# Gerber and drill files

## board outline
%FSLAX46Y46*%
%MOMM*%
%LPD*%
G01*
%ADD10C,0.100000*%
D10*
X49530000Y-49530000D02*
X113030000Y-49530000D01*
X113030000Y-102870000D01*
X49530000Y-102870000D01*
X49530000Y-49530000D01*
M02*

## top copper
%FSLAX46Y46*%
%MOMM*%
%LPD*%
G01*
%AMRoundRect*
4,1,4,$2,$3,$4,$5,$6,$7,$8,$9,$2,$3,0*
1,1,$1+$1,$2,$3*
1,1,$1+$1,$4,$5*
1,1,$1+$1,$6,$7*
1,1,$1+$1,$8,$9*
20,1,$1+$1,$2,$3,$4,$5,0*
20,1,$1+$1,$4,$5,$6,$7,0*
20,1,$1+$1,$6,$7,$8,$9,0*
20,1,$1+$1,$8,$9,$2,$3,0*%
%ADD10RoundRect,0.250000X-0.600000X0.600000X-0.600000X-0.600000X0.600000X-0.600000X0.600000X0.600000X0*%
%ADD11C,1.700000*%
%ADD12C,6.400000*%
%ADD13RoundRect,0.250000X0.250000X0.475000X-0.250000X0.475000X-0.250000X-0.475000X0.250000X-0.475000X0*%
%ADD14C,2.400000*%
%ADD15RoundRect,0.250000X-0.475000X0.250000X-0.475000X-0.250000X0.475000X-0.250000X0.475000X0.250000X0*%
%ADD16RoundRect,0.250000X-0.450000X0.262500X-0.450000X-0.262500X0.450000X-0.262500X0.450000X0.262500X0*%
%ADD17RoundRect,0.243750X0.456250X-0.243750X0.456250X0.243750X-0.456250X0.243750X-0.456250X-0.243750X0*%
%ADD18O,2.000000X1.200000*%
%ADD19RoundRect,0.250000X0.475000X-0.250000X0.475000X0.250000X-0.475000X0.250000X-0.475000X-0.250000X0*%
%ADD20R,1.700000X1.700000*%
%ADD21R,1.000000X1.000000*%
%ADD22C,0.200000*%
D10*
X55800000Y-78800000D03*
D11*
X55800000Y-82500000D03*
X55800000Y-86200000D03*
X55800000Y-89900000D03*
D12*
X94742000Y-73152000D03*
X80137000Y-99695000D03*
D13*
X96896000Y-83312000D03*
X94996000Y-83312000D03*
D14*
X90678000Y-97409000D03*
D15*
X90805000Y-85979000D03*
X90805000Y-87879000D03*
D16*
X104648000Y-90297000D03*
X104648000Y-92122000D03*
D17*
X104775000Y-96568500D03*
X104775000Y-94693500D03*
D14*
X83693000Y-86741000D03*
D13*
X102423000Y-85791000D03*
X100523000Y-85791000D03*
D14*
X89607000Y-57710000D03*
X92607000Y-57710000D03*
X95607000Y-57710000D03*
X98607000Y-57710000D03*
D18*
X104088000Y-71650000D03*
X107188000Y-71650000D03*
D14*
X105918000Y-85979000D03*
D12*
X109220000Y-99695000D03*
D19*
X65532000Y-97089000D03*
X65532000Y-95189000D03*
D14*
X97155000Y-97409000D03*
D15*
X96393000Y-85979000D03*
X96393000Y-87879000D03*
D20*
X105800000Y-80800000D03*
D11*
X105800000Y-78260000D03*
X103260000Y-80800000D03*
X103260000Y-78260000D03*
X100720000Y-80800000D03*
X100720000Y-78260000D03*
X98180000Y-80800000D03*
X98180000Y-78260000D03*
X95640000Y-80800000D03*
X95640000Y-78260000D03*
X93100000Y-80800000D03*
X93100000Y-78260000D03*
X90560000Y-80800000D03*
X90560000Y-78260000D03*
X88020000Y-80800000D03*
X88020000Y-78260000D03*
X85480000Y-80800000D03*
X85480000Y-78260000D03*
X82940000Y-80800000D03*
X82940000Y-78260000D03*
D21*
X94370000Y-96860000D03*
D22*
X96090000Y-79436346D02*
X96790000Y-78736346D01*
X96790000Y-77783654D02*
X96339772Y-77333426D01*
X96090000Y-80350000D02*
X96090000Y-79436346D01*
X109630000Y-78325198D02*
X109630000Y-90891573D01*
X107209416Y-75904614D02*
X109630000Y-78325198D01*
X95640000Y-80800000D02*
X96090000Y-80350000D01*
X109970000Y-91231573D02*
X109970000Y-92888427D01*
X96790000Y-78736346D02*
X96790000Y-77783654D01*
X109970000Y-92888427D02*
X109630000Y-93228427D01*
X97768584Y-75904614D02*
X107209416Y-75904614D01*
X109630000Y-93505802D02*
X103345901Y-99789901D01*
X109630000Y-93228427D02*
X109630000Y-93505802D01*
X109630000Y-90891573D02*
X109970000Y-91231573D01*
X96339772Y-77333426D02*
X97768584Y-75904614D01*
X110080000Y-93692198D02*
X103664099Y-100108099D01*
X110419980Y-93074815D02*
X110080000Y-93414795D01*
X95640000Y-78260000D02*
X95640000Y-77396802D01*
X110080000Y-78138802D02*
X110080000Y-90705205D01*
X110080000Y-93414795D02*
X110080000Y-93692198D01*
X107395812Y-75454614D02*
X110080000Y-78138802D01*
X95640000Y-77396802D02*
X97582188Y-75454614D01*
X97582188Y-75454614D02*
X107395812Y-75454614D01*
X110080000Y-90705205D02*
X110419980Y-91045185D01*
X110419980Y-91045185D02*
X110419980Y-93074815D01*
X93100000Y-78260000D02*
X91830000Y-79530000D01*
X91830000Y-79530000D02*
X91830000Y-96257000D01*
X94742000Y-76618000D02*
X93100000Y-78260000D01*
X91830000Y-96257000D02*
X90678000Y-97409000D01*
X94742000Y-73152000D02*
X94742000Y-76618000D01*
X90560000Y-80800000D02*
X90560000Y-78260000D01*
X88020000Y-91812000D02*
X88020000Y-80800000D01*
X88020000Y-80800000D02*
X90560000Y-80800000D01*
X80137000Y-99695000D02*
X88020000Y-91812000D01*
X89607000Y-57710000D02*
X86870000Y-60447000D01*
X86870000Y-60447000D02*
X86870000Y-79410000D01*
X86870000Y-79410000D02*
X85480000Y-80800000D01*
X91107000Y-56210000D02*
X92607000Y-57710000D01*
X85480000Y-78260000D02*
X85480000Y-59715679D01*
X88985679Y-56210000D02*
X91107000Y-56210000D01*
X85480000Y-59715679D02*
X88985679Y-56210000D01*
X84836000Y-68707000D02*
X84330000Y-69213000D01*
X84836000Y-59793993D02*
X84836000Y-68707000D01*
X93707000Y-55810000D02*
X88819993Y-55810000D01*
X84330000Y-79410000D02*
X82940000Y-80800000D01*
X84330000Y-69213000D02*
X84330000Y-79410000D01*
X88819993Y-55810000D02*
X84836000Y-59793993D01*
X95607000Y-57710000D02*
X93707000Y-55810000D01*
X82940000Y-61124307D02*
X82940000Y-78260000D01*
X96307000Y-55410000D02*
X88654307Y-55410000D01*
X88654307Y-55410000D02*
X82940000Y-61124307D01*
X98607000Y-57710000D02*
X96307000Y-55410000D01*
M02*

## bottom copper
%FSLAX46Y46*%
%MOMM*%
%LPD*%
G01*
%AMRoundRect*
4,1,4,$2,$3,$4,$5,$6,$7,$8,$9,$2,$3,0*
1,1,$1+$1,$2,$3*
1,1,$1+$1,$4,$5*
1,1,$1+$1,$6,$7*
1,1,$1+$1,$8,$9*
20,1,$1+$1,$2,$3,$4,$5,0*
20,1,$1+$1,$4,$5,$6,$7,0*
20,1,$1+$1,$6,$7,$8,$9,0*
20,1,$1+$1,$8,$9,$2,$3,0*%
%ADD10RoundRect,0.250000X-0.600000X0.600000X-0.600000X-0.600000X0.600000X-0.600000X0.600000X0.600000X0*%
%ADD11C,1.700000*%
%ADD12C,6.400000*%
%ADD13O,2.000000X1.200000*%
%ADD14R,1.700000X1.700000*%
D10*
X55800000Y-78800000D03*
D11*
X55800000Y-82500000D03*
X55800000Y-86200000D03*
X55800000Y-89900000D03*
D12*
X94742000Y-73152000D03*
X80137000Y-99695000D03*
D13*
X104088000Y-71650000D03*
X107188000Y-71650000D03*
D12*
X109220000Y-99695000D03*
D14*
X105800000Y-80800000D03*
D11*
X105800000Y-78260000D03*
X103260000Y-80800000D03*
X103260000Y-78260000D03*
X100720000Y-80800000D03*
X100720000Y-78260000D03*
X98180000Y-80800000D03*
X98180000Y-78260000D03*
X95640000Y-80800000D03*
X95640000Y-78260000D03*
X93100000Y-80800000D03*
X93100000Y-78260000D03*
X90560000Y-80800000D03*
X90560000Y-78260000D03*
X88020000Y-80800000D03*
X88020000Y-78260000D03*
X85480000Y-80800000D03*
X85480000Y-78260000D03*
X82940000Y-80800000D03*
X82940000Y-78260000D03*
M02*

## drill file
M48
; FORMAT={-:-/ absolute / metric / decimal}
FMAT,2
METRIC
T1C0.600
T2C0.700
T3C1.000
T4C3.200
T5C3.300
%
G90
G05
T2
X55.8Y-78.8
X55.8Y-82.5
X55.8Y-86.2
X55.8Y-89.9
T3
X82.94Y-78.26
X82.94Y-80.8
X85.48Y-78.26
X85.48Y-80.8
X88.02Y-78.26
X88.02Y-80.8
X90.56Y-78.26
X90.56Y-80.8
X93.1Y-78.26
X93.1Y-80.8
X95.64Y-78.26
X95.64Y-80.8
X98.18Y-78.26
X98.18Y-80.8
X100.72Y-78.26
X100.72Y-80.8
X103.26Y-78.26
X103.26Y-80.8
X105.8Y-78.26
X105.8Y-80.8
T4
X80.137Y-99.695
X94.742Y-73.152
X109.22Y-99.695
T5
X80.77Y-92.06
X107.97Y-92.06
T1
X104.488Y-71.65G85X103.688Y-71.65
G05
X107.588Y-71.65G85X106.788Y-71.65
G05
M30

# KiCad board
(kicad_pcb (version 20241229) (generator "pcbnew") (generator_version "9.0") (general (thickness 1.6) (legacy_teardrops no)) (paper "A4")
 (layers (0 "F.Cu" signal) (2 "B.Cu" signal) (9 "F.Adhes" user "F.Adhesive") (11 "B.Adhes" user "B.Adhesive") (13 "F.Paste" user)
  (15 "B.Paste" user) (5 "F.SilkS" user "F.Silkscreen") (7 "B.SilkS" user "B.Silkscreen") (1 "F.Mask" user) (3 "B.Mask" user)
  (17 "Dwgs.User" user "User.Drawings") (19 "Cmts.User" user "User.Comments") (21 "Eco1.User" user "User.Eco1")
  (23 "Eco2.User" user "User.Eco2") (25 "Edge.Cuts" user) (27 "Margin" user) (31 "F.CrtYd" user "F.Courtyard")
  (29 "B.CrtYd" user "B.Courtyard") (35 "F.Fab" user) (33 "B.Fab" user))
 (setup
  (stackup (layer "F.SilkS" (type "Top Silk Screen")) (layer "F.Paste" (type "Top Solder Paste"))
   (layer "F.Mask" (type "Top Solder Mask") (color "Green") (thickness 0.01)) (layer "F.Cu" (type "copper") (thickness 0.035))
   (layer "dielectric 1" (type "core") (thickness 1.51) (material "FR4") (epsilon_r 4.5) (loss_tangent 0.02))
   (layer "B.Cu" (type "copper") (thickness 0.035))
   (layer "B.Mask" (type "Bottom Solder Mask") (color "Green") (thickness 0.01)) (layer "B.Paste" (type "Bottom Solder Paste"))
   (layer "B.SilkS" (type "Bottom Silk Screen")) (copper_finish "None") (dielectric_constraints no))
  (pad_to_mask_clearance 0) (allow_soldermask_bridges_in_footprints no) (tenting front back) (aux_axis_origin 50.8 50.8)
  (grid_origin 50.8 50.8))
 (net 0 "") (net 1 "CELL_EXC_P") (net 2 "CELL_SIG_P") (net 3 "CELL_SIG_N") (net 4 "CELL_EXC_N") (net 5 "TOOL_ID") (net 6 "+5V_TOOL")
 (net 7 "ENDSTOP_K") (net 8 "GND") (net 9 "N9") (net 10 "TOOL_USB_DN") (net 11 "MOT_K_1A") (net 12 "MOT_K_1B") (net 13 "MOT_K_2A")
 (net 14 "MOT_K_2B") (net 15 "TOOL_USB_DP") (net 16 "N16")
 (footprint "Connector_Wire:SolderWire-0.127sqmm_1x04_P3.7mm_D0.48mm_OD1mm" (layer "F.Cu") (at 55.8 78.8 -90)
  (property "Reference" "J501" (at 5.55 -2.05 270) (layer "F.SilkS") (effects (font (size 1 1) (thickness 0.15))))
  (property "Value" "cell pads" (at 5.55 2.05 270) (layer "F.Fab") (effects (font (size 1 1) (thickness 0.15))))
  (pad "1" thru_hole roundrect (at 0 0 270) (size 1.7 1.7) (drill 0.7) (layers "*.Cu" "*.Mask") (remove_unused_layers no)
   (roundrect_rratio 0.147059) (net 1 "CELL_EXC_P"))
  (pad "2" thru_hole circle (at 3.7 0 270) (size 1.7 1.7) (drill 0.7) (layers "*.Cu" "*.Mask") (remove_unused_layers no)
   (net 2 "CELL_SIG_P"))
  (pad "3" thru_hole circle (at 7.4 0 270) (size 1.7 1.7) (drill 0.7) (layers "*.Cu" "*.Mask") (remove_unused_layers no)
   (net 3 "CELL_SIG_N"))
  (pad "4" thru_hole circle (at 11.1 0 270) (size 1.7 1.7) (drill 0.7) (layers "*.Cu" "*.Mask") (remove_unused_layers no)
   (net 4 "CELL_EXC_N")))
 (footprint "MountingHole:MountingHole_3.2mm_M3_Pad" (layer "F.Cu") (at 94.742 73.152)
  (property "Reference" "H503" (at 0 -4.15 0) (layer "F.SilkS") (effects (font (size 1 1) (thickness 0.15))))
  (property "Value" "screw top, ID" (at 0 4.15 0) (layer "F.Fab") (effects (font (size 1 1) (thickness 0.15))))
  (pad "1" thru_hole circle (at 0 0) (size 6.4 6.4) (drill 3.2) (layers "*.Cu" "*.Mask") (remove_unused_layers no) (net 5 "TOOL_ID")
   (zone_connect 2)))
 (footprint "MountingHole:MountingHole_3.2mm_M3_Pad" (layer "F.Cu") (at 80.137 99.695)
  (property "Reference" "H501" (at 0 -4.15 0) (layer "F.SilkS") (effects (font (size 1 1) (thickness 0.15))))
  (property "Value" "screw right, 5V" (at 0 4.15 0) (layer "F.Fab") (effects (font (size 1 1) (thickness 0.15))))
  (pad "1" thru_hole circle (at 0 0) (size 6.4 6.4) (drill 3.2) (layers "*.Cu" "*.Mask") (remove_unused_layers no) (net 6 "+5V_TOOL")
   (zone_connect 2)))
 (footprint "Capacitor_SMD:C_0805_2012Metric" (layer "F.Cu") (at 95.946 83.312 180)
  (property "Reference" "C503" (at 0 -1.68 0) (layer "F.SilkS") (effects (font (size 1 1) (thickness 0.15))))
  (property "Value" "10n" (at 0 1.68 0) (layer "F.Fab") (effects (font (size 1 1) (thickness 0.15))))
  (pad "1" smd roundrect (at -0.95 0 180) (size 1 1.45) (layers "F.Cu" "F.Mask" "F.Paste") (roundrect_rratio 0.25) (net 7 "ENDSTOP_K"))
  (pad "2" smd roundrect (at 0.95 0 180) (size 1 1.45) (layers "F.Cu" "F.Mask" "F.Paste") (roundrect_rratio 0.25) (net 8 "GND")))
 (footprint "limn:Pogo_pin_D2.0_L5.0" (layer "F.Cu") (at 90.678 97.409)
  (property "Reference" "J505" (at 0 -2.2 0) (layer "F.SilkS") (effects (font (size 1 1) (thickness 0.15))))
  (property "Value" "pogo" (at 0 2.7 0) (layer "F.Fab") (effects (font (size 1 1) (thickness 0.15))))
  (pad "1" smd circle (at 0 0) (size 2.4 2.4) (layers "F.Cu" "F.Mask" "F.Paste") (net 5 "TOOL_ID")))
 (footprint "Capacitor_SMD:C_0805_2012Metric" (layer "F.Cu") (at 90.805 86.929 -90)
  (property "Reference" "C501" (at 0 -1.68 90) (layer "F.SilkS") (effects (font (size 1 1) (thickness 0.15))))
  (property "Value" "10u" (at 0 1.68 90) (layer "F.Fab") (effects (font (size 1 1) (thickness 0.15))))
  (pad "1" smd roundrect (at -0.95 0 270) (size 1 1.45) (layers "F.Cu" "F.Mask" "F.Paste") (roundrect_rratio 0.25) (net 6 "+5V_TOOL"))
  (pad "2" smd roundrect (at 0.95 0 270) (size 1 1.45) (layers "F.Cu" "F.Mask" "F.Paste") (roundrect_rratio 0.25) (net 8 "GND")))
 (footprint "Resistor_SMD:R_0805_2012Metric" (layer "F.Cu") (at 104.648 91.2095 -90)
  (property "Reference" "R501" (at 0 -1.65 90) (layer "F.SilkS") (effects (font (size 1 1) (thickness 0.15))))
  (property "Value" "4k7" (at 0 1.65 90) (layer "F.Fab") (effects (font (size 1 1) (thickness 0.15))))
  (pad "1" smd roundrect (at -0.9125 0 270) (size 1.025 1.4) (layers "F.Cu" "F.Mask" "F.Paste") (roundrect_rratio 0.243902)
   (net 6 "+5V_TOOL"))
  (pad "2" smd roundrect (at 0.9125 0 270) (size 1.025 1.4) (layers "F.Cu" "F.Mask" "F.Paste") (roundrect_rratio 0.243902) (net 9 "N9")))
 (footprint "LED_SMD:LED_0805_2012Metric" (layer "F.Cu") (at 104.775 95.631 90)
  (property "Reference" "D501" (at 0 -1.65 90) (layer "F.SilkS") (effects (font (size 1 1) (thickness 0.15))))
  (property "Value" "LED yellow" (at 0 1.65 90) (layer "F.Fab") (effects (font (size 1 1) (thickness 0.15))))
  (pad "1" smd roundrect (at -0.9375 0 90) (size 0.975 1.4) (layers "F.Cu" "F.Mask" "F.Paste") (roundrect_rratio 0.25) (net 8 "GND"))
  (pad "2" smd roundrect (at 0.9375 0 90) (size 0.975 1.4) (layers "F.Cu" "F.Mask" "F.Paste") (roundrect_rratio 0.25) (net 9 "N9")))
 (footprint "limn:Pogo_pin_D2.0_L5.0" (layer "F.Cu") (at 83.693 86.741)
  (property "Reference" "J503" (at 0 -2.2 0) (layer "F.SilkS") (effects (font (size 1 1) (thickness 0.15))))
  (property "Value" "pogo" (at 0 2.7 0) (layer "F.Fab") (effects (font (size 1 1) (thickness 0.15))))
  (pad "1" smd circle (at 0 0) (size 2.4 2.4) (layers "F.Cu" "F.Mask" "F.Paste") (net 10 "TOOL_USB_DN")))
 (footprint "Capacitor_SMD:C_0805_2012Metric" (layer "F.Cu") (at 101.473 85.791 180)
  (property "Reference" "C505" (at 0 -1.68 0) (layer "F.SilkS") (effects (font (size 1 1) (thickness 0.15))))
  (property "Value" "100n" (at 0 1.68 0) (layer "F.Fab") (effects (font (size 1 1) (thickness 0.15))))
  (pad "1" smd roundrect (at -0.95 0 180) (size 1 1.45) (layers "F.Cu" "F.Mask" "F.Paste") (roundrect_rratio 0.25) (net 1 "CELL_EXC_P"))
  (pad "2" smd roundrect (at 0.95 0 180) (size 1 1.45) (layers "F.Cu" "F.Mask" "F.Paste") (roundrect_rratio 0.25) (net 4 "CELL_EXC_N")))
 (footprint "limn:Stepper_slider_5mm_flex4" (layer "F.Cu") (at 94.107 67.21 90)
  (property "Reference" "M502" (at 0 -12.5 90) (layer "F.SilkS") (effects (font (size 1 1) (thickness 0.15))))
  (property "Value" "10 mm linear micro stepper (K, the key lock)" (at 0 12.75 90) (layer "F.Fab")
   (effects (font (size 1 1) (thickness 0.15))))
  (pad "1" smd circle (at 9.5 -4.5 90) (size 2.4 2.4) (layers "F.Cu" "F.Mask" "F.Paste") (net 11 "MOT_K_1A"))
  (pad "2" smd circle (at 9.5 -1.5 90) (size 2.4 2.4) (layers "F.Cu" "F.Mask" "F.Paste") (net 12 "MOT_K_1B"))
  (pad "3" smd circle (at 9.5 1.5 90) (size 2.4 2.4) (layers "F.Cu" "F.Mask" "F.Paste") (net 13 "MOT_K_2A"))
  (pad "4" smd circle (at 9.5 4.5 90) (size 2.4 2.4) (layers "F.Cu" "F.Mask" "F.Paste") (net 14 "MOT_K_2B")))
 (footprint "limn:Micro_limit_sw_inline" (layer "F.Cu") (at 107.188 69.85 -90)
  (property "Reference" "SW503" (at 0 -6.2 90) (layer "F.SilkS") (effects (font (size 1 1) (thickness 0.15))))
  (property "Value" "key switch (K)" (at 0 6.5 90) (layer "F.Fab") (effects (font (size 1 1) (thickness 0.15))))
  (pad "1" thru_hole oval (at 1.8 3.1 270) (size 1.2 2) (drill oval 0.6 1.4) (layers "*.Cu" "*.Mask") (remove_unused_layers no)
   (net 7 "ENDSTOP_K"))
  (pad "2" thru_hole oval (at 1.8 0 270) (size 1.2 2) (drill oval 0.6 1.4) (layers "*.Cu" "*.Mask") (remove_unused_layers no) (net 8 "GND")))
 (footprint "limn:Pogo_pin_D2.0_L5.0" (layer "F.Cu") (at 105.918 85.979)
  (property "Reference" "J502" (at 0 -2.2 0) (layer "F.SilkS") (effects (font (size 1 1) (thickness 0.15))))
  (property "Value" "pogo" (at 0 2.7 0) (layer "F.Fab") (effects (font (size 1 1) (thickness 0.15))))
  (pad "1" smd circle (at 0 0) (size 2.4 2.4) (layers "F.Cu" "F.Mask" "F.Paste") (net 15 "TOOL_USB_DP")))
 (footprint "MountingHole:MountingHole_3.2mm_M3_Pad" (layer "F.Cu") (at 109.22 99.695)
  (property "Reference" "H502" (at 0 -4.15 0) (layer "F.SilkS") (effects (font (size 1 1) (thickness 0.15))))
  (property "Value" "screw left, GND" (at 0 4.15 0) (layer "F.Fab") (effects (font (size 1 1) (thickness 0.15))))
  (pad "1" thru_hole circle (at 0 0) (size 6.4 6.4) (drill 3.2) (layers "*.Cu" "*.Mask") (remove_unused_layers no) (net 8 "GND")
   (zone_connect 2)))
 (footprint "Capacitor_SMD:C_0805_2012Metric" (layer "F.Cu") (at 65.532 96.139 90)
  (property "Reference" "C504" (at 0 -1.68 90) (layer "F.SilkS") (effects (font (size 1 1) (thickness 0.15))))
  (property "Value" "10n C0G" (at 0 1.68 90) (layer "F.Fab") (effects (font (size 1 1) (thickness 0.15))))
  (pad "1" smd roundrect (at -0.95 0 90) (size 1 1.45) (layers "F.Cu" "F.Mask" "F.Paste") (roundrect_rratio 0.25) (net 2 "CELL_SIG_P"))
  (pad "2" smd roundrect (at 0.95 0 90) (size 1 1.45) (layers "F.Cu" "F.Mask" "F.Paste") (roundrect_rratio 0.25) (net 3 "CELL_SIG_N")))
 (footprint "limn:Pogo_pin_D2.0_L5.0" (layer "F.Cu") (at 97.155 97.409)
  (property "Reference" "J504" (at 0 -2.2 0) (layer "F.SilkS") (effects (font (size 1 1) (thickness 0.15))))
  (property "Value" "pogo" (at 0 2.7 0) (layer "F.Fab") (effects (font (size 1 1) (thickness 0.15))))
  (pad "1" smd circle (at 0 0) (size 2.4 2.4) (layers "F.Cu" "F.Mask" "F.Paste") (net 8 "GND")))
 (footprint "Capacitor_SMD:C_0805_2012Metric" (layer "F.Cu") (at 96.393 86.929 -90)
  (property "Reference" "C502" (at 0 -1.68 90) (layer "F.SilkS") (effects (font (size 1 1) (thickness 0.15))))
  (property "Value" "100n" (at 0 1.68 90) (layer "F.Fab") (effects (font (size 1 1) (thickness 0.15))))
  (pad "1" smd roundrect (at -0.95 0 270) (size 1 1.45) (layers "F.Cu" "F.Mask" "F.Paste") (roundrect_rratio 0.25) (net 6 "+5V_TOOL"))
  (pad "2" smd roundrect (at 0.95 0 270) (size 1 1.45) (layers "F.Cu" "F.Mask" "F.Paste") (roundrect_rratio 0.25) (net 8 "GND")))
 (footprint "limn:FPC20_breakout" (layer "F.Cu") (at 105.8 80.8)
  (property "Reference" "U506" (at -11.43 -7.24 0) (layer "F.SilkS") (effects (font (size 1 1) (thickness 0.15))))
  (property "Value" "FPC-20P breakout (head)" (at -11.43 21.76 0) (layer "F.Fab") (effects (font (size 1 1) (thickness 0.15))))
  (pad "" np_thru_hole circle (at -25.03 11.26) (size 3.3 3.3) (drill 3.3) (layers "*.Cu" "*.Mask"))
  (pad "" np_thru_hole circle (at 2.17 11.26) (size 3.3 3.3) (drill 3.3) (layers "*.Cu" "*.Mask"))
  (pad "1" thru_hole rect (at 0 0) (size 1.7 1.7) (drill 1) (layers "*.Cu" "*.Mask") (remove_unused_layers no) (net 8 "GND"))
  (pad "2" thru_hole circle (at 0 -2.54) (size 1.7 1.7) (drill 1) (layers "*.Cu" "*.Mask") (remove_unused_layers no) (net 1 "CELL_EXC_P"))
  (pad "3" thru_hole circle (at -2.54 0) (size 1.7 1.7) (drill 1) (layers "*.Cu" "*.Mask") (remove_unused_layers no) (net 2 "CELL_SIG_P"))
  (pad "4" thru_hole circle (at -2.54 -2.54) (size 1.7 1.7) (drill 1) (layers "*.Cu" "*.Mask") (remove_unused_layers no)
   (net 3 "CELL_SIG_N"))
  (pad "5" thru_hole circle (at -5.08 0) (size 1.7 1.7) (drill 1) (layers "*.Cu" "*.Mask") (remove_unused_layers no) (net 4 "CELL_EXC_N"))
  (pad "6" thru_hole circle (at -5.08 -2.54) (size 1.7 1.7) (drill 1) (layers "*.Cu" "*.Mask") (remove_unused_layers no) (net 8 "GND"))
  (pad "7" thru_hole circle (at -7.62 0) (size 1.7 1.7) (drill 1) (layers "*.Cu" "*.Mask") (remove_unused_layers no) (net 7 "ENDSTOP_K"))
  (pad "8" thru_hole circle (at -7.62 -2.54) (size 1.7 1.7) (drill 1) (layers "*.Cu" "*.Mask") (remove_unused_layers no) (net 8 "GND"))
  (pad "9" thru_hole circle (at -10.16 0) (size 1.7 1.7) (drill 1) (layers "*.Cu" "*.Mask") (remove_unused_layers no) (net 15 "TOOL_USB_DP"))
  (pad "10" thru_hole circle (at -10.16 -2.54) (size 1.7 1.7) (drill 1) (layers "*.Cu" "*.Mask") (remove_unused_layers no)
   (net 10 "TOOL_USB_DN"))
  (pad "11" thru_hole circle (at -12.7 0) (size 1.7 1.7) (drill 1) (layers "*.Cu" "*.Mask") (remove_unused_layers no) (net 8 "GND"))
  (pad "12" thru_hole circle (at -12.7 -2.54) (size 1.7 1.7) (drill 1) (layers "*.Cu" "*.Mask") (remove_unused_layers no) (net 5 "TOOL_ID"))
  (pad "13" thru_hole circle (at -15.24 0) (size 1.7 1.7) (drill 1) (layers "*.Cu" "*.Mask") (remove_unused_layers no) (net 6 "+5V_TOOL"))
  (pad "14" thru_hole circle (at -15.24 -2.54) (size 1.7 1.7) (drill 1) (layers "*.Cu" "*.Mask") (remove_unused_layers no)
   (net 6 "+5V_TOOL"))
  (pad "15" thru_hole circle (at -17.78 0) (size 1.7 1.7) (drill 1) (layers "*.Cu" "*.Mask") (remove_unused_layers no) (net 6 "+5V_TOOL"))
  (pad "16" thru_hole circle (at -17.78 -2.54) (size 1.7 1.7) (drill 1) (layers "*.Cu" "*.Mask") (remove_unused_layers no) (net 8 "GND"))
  (pad "17" thru_hole circle (at -20.32 0) (size 1.7 1.7) (drill 1) (layers "*.Cu" "*.Mask") (remove_unused_layers no) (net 11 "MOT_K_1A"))
  (pad "18" thru_hole circle (at -20.32 -2.54) (size 1.7 1.7) (drill 1) (layers "*.Cu" "*.Mask") (remove_unused_layers no)
   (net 12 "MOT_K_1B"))
  (pad "19" thru_hole circle (at -22.86 0) (size 1.7 1.7) (drill 1) (layers "*.Cu" "*.Mask") (remove_unused_layers no) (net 13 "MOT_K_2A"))
  (pad "20" thru_hole circle (at -22.86 -2.54) (size 1.7 1.7) (drill 1) (layers "*.Cu" "*.Mask") (remove_unused_layers no)
   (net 14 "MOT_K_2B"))
  (pad "21" smd rect (at -11.43 16.06) (size 1 1) (layers "F.Cu" "F.Mask") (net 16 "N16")))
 (gr_rect (start 49.53 49.53) (end 113.03 102.87) (stroke (width 0.1) (type solid)) (fill no) (layer "Edge.Cuts"))
 (segment (start 96.09 79.436346) (end 96.79 78.736346) (width 0.2) (layer "F.Cu") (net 15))
 (segment (start 96.79 77.783654) (end 96.339772 77.333426) (width 0.2) (layer "F.Cu") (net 15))
 (segment (start 96.09 80.35) (end 96.09 79.436346) (width 0.2) (layer "F.Cu") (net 15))
 (segment (start 109.63 78.325198) (end 109.63 90.891573) (width 0.2) (layer "F.Cu") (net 15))
 (segment (start 107.209416 75.904614) (end 109.63 78.325198) (width 0.2) (layer "F.Cu") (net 15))
 (segment (start 95.64 80.8) (end 96.09 80.35) (width 0.2) (layer "F.Cu") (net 15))
 (segment (start 109.97 91.231573) (end 109.97 92.888427) (width 0.2) (layer "F.Cu") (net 15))
 (segment (start 96.79 78.736346) (end 96.79 77.783654) (width 0.2) (layer "F.Cu") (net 15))
 (segment (start 109.97 92.888427) (end 109.63 93.228427) (width 0.2) (layer "F.Cu") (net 15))
 (segment (start 97.768584 75.904614) (end 107.209416 75.904614) (width 0.2) (layer "F.Cu") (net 15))
 (segment (start 109.63 93.505802) (end 103.345901 99.789901) (width 0.2) (layer "F.Cu") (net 15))
 (segment (start 109.63 93.228427) (end 109.63 93.505802) (width 0.2) (layer "F.Cu") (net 15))
 (segment (start 109.63 90.891573) (end 109.97 91.231573) (width 0.2) (layer "F.Cu") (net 15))
 (segment (start 96.339772 77.333426) (end 97.768584 75.904614) (width 0.2) (layer "F.Cu") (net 15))
 (segment (start 110.08 93.692198) (end 103.664099 100.108099) (width 0.2) (layer "F.Cu") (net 10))
 (segment (start 110.41998 93.074815) (end 110.08 93.414795) (width 0.2) (layer "F.Cu") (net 10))
 (segment (start 95.64 78.26) (end 95.64 77.396802) (width 0.2) (layer "F.Cu") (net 10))
 (segment (start 110.08 78.138802) (end 110.08 90.705205) (width 0.2) (layer "F.Cu") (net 10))
 (segment (start 110.08 93.414795) (end 110.08 93.692198) (width 0.2) (layer "F.Cu") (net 10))
 (segment (start 107.395812 75.454614) (end 110.08 78.138802) (width 0.2) (layer "F.Cu") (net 10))
 (segment (start 95.64 77.396802) (end 97.582188 75.454614) (width 0.2) (layer "F.Cu") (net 10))
 (segment (start 97.582188 75.454614) (end 107.395812 75.454614) (width 0.2) (layer "F.Cu") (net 10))
 (segment (start 110.08 90.705205) (end 110.41998 91.045185) (width 0.2) (layer "F.Cu") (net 10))
 (segment (start 110.41998 91.045185) (end 110.41998 93.074815) (width 0.2) (layer "F.Cu") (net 10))
 (segment (start 93.1 78.26) (end 91.83 79.53) (width 0.2) (layer "F.Cu") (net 5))
 (segment (start 91.83 79.53) (end 91.83 96.257) (width 0.2) (layer "F.Cu") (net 5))
 (segment (start 94.742 76.618) (end 93.1 78.26) (width 0.2) (layer "F.Cu") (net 5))
 (segment (start 91.83 96.257) (end 90.678 97.409) (width 0.2) (layer "F.Cu") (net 5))
 (segment (start 94.742 73.152) (end 94.742 76.618) (width 0.2) (layer "F.Cu") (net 5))
 (segment (start 90.56 80.8) (end 90.56 78.26) (width 0.2) (layer "F.Cu") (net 6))
 (segment (start 88.02 91.812) (end 88.02 80.8) (width 0.2) (layer "F.Cu") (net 6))
 (segment (start 88.02 80.8) (end 90.56 80.8) (width 0.2) (layer "F.Cu") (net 6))
 (segment (start 80.137 99.695) (end 88.02 91.812) (width 0.2) (layer "F.Cu") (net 6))
 (segment (start 89.607 57.71) (end 86.87 60.447) (width 0.2) (layer "F.Cu") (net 11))
 (segment (start 86.87 60.447) (end 86.87 79.41) (width 0.2) (layer "F.Cu") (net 11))
 (segment (start 86.87 79.41) (end 85.48 80.8) (width 0.2) (layer "F.Cu") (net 11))
 (segment (start 91.107 56.21) (end 92.607 57.71) (width 0.2) (layer "F.Cu") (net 12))
 (segment (start 85.48 78.26) (end 85.48 59.715679) (width 0.2) (layer "F.Cu") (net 12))
 (segment (start 88.985679 56.21) (end 91.107 56.21) (width 0.2) (layer "F.Cu") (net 12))
 (segment (start 85.48 59.715679) (end 88.985679 56.21) (width 0.2) (layer "F.Cu") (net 12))
 (segment (start 84.836 68.707) (end 84.33 69.213) (width 0.2) (layer "F.Cu") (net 13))
 (segment (start 84.836 59.793993) (end 84.836 68.707) (width 0.2) (layer "F.Cu") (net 13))
 (segment (start 93.707 55.81) (end 88.819993 55.81) (width 0.2) (layer "F.Cu") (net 13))
 (segment (start 84.33 79.41) (end 82.94 80.8) (width 0.2) (layer "F.Cu") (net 13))
 (segment (start 84.33 69.213) (end 84.33 79.41) (width 0.2) (layer "F.Cu") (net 13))
 (segment (start 88.819993 55.81) (end 84.836 59.793993) (width 0.2) (layer "F.Cu") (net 13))
 (segment (start 95.607 57.71) (end 93.707 55.81) (width 0.2) (layer "F.Cu") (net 13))
 (segment (start 82.94 61.124307) (end 82.94 78.26) (width 0.2) (layer "F.Cu") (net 14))
 (segment (start 96.307 55.41) (end 88.654307 55.41) (width 0.2) (layer "F.Cu") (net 14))
 (segment (start 88.654307 55.41) (end 82.94 61.124307) (width 0.2) (layer "F.Cu") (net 14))
 (segment (start 98.607 57.71) (end 96.307 55.41) (width 0.2) (layer "F.Cu") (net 14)))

